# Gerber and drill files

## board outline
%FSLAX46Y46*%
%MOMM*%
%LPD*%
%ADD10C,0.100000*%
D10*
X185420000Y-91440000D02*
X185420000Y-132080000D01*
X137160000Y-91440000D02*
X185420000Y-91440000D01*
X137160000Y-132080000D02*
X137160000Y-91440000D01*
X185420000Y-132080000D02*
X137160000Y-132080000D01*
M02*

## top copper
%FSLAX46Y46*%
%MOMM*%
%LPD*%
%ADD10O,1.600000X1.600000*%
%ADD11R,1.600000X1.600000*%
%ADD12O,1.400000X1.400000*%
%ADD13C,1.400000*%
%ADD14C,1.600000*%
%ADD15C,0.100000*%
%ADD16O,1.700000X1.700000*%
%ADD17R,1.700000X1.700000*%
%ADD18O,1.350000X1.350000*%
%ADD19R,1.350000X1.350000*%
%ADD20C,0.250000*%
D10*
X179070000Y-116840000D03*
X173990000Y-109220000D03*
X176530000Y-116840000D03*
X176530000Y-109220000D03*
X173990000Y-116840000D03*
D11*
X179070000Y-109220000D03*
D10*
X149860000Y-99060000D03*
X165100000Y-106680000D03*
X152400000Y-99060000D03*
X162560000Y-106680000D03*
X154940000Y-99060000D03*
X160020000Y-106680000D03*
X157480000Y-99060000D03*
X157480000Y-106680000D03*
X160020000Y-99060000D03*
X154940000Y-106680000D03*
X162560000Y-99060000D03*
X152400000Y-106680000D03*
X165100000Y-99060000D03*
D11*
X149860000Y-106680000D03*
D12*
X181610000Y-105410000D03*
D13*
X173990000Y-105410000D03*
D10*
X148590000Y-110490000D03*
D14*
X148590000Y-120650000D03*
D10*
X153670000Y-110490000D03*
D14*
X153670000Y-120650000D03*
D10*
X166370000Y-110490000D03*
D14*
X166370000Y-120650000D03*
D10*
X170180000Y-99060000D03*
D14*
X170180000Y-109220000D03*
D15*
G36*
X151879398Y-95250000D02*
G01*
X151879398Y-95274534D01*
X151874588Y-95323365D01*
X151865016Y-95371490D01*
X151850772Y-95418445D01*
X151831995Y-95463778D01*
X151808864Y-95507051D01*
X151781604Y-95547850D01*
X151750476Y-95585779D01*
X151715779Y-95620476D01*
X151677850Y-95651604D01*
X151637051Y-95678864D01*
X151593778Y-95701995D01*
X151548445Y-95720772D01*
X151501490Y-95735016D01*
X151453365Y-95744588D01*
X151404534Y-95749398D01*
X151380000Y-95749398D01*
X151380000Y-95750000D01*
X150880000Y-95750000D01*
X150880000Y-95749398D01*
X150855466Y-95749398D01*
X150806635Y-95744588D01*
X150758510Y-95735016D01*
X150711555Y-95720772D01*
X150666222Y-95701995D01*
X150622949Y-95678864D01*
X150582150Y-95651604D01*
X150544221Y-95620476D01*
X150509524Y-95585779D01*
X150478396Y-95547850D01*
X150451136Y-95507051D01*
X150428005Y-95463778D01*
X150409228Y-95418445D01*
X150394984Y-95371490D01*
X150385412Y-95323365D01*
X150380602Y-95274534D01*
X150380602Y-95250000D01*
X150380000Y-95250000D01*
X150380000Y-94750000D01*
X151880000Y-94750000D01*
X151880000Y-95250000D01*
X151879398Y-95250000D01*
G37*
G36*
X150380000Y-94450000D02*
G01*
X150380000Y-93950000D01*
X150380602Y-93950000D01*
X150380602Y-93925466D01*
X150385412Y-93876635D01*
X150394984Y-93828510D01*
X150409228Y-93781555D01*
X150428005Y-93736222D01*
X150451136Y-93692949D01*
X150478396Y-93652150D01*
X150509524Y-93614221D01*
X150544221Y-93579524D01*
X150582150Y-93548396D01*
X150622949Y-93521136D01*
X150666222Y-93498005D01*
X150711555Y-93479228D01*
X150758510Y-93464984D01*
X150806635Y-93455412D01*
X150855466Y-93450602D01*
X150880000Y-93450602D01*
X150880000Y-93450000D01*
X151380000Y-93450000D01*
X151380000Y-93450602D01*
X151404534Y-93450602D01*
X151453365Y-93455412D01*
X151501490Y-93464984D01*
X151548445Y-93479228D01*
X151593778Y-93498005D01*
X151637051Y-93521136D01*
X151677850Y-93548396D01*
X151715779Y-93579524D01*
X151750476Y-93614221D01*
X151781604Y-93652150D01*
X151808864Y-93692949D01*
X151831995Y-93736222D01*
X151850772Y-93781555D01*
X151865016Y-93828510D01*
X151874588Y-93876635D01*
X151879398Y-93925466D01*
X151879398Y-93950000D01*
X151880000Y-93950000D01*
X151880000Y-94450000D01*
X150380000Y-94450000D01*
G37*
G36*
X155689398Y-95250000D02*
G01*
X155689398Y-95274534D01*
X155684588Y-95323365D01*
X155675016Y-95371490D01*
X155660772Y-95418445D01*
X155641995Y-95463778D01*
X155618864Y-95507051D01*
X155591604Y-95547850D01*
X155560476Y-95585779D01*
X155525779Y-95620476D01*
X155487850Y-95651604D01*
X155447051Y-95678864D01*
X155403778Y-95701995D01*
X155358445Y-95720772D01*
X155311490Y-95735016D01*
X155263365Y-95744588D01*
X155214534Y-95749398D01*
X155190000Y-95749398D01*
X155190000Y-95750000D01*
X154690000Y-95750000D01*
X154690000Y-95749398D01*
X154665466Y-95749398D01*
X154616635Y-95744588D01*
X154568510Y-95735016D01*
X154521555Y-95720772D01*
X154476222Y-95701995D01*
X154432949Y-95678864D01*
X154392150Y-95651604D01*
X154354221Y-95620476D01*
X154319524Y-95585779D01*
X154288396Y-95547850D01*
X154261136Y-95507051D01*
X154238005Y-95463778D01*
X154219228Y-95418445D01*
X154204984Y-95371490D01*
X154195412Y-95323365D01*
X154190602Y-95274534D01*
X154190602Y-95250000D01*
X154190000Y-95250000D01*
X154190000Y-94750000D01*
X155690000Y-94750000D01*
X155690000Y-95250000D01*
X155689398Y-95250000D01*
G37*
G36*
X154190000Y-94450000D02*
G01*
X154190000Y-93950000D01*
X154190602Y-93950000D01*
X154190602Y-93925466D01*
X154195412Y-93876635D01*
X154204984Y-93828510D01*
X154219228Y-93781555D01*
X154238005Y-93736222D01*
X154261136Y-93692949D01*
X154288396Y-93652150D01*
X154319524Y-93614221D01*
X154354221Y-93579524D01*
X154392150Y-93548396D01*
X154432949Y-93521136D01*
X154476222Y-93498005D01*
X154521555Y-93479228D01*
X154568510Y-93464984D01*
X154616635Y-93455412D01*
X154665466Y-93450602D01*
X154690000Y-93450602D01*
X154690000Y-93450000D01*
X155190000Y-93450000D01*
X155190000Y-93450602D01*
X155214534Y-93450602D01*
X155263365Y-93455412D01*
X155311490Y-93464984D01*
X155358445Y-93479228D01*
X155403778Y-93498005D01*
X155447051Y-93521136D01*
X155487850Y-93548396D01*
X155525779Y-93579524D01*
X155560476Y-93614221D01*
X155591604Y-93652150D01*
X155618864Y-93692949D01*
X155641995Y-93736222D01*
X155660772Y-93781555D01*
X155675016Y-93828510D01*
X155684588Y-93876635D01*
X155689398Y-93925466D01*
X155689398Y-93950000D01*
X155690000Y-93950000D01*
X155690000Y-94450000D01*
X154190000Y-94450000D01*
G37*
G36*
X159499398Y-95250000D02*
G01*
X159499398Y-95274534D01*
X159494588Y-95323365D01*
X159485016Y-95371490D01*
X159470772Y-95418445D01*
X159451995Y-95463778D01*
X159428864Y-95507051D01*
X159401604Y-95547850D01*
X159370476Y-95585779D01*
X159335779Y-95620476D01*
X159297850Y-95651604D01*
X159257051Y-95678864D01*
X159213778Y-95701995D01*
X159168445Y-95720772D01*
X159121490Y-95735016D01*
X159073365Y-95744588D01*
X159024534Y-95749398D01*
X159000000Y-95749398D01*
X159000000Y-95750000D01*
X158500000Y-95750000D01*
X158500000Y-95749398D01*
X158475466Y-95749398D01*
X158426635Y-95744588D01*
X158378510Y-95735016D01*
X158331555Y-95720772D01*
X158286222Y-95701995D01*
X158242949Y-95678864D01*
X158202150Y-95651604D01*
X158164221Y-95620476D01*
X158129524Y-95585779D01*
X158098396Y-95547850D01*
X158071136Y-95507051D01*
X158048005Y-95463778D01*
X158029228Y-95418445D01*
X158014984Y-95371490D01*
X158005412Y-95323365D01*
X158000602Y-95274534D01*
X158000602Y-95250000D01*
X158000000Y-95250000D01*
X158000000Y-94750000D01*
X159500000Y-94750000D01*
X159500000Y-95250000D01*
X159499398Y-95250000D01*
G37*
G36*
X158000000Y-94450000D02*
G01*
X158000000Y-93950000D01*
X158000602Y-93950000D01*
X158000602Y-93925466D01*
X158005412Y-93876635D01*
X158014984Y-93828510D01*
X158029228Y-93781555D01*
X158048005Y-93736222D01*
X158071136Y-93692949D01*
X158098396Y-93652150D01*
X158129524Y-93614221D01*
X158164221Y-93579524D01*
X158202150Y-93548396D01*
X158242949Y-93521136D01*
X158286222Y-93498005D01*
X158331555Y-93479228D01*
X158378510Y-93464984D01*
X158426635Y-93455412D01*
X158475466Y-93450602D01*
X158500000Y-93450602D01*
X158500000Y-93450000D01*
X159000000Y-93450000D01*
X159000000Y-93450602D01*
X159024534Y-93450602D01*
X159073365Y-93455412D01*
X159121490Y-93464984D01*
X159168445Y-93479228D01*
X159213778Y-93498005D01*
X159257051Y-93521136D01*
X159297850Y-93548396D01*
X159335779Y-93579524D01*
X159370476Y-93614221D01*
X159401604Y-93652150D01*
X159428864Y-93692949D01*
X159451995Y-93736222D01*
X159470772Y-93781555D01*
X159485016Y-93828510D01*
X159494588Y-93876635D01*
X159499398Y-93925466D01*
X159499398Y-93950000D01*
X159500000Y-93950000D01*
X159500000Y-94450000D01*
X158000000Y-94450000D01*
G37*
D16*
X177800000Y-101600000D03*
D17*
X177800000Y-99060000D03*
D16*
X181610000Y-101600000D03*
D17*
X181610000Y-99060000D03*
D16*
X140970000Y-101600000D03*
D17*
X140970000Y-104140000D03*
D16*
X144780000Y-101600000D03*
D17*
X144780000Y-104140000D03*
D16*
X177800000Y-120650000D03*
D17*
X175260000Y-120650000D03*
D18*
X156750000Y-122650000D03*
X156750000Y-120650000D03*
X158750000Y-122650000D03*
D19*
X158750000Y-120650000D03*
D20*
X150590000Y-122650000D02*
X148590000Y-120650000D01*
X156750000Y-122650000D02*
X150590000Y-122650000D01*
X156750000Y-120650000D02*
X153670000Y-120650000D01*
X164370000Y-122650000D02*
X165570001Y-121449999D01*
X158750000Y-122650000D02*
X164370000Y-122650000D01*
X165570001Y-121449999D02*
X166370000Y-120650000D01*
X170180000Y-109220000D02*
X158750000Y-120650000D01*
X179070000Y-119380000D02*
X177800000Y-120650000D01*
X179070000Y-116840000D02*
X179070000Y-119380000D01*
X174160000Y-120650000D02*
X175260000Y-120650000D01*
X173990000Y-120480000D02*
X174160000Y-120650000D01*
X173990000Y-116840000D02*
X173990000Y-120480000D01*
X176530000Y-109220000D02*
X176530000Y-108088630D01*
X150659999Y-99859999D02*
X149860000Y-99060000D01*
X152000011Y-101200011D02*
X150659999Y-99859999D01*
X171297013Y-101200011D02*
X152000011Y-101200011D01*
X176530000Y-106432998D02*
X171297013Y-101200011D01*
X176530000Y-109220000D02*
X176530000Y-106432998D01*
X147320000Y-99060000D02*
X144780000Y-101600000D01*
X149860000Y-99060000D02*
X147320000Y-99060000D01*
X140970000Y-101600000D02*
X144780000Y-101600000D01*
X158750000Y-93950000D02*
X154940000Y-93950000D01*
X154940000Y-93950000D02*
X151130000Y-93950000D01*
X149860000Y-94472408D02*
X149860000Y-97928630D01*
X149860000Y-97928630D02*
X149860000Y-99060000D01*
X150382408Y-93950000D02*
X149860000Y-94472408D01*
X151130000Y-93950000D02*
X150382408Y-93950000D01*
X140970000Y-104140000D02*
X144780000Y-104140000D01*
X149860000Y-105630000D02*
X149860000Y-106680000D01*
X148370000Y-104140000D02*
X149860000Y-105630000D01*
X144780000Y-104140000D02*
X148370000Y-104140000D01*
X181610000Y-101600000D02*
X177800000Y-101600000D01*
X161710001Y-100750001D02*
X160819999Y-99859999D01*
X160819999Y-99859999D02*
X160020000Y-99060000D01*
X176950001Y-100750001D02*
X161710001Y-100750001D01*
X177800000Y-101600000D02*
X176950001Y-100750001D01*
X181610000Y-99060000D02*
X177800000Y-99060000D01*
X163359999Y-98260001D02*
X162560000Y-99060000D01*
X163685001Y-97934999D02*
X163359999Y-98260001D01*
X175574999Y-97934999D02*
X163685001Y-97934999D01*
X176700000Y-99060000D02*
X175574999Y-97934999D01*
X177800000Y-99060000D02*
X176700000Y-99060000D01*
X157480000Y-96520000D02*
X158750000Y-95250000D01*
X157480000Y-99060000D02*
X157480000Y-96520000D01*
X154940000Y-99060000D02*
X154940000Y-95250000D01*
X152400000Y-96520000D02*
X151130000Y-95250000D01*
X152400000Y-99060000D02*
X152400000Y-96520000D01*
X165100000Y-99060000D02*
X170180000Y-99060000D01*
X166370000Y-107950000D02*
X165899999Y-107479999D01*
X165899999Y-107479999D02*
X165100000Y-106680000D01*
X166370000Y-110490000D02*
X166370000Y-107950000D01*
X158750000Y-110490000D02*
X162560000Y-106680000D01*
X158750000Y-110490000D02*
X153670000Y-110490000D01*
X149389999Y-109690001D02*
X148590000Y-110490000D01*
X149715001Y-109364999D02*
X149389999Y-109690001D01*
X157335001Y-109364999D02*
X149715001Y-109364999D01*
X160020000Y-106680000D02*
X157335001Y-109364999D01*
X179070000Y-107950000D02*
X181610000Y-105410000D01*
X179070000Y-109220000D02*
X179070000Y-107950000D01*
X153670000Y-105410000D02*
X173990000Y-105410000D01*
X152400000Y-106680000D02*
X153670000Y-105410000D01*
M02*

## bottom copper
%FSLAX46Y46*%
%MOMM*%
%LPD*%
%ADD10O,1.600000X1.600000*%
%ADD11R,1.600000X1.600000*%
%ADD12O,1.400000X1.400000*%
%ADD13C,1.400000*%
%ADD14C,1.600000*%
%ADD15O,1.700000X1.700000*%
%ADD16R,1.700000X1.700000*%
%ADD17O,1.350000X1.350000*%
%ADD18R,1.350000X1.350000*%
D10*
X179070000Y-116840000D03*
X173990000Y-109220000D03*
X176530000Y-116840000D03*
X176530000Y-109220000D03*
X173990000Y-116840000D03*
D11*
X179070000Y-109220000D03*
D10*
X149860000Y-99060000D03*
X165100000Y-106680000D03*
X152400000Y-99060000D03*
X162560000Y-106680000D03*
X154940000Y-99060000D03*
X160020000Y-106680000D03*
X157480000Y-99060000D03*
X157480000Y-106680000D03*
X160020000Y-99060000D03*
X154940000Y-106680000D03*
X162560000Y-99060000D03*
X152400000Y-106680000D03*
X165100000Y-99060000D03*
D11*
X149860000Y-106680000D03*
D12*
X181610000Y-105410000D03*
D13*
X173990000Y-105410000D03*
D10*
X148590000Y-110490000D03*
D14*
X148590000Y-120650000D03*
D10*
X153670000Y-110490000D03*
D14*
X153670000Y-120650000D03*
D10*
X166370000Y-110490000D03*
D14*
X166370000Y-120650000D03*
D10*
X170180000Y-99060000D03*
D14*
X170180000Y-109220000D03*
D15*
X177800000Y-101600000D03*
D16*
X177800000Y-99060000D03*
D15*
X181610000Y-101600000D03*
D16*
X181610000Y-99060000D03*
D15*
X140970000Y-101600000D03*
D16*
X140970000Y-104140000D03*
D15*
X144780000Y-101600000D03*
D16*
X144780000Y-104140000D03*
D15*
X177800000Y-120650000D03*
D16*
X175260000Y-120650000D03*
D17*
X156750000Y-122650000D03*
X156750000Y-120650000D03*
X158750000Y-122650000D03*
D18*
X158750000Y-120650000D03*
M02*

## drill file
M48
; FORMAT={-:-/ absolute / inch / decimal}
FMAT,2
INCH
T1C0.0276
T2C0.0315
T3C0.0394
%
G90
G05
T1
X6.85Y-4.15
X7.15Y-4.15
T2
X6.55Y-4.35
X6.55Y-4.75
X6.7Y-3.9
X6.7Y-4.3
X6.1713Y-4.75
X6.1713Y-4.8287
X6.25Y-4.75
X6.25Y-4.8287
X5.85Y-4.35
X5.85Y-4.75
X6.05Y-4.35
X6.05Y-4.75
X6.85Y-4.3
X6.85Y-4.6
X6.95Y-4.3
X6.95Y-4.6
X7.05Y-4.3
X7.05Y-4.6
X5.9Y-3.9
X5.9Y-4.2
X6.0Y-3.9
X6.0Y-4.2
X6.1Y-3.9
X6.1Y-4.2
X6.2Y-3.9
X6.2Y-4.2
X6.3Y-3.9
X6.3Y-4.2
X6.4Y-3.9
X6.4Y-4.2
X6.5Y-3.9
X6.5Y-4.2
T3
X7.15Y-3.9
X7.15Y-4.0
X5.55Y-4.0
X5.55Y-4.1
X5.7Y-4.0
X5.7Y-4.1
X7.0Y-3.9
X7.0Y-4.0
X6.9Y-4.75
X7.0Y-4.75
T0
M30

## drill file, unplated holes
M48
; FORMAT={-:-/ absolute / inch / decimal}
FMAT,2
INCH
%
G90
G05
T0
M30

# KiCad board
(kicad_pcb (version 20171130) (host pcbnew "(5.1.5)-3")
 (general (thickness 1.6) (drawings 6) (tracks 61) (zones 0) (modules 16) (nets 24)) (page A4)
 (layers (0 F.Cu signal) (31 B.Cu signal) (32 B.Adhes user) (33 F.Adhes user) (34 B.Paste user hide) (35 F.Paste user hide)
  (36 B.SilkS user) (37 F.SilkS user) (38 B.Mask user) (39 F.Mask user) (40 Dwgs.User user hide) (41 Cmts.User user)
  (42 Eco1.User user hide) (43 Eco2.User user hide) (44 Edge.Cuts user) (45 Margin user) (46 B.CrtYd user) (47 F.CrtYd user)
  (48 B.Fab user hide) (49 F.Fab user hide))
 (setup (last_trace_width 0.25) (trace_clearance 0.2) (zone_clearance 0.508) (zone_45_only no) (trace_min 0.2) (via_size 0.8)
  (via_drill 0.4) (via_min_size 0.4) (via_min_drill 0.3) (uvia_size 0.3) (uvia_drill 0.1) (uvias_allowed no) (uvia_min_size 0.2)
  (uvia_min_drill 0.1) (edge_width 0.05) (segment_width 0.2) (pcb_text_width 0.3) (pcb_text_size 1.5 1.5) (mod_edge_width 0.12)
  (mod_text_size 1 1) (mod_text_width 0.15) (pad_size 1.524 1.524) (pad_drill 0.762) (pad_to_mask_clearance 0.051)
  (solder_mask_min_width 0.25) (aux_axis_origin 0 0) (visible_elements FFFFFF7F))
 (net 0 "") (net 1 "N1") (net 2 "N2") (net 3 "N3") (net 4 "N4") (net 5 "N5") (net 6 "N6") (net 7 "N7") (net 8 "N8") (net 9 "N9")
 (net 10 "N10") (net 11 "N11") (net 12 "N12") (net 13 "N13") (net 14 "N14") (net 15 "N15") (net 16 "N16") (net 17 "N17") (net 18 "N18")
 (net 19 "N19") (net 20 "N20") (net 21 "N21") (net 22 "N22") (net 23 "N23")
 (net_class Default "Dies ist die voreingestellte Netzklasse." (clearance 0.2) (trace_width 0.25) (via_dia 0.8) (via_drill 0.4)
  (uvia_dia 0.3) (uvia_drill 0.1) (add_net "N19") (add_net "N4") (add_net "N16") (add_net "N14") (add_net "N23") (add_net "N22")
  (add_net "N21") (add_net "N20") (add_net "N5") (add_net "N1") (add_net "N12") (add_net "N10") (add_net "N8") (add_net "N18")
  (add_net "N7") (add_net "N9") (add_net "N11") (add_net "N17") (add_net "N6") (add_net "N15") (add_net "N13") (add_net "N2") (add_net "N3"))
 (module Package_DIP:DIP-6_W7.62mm (layer F.Cu) (at 179.07 109.22 270)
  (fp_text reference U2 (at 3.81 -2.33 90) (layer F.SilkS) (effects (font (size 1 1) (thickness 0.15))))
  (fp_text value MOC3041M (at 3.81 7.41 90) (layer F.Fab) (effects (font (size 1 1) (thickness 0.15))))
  (pad 6 thru_hole oval (at 7.62 0 270) (size 1.6 1.6) (drill 0.8) (layers *.Cu *.Mask) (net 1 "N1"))
  (pad 3 thru_hole oval (at 0 5.08 270) (size 1.6 1.6) (drill 0.8) (layers *.Cu *.Mask) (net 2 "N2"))
  (pad 5 thru_hole oval (at 7.62 2.54 270) (size 1.6 1.6) (drill 0.8) (layers *.Cu *.Mask) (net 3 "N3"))
  (pad 2 thru_hole oval (at 0 2.54 270) (size 1.6 1.6) (drill 0.8) (layers *.Cu *.Mask) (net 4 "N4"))
  (pad 4 thru_hole oval (at 7.62 5.08 270) (size 1.6 1.6) (drill 0.8) (layers *.Cu *.Mask) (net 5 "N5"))
  (pad 1 thru_hole rect (at 0 0 270) (size 1.6 1.6) (drill 0.8) (layers *.Cu *.Mask) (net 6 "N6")))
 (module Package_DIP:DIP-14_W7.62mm (layer F.Cu) (at 149.86 106.68 90)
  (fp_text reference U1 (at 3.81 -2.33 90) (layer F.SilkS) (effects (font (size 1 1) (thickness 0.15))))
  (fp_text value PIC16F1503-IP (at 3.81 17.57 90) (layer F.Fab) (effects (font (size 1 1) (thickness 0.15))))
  (pad 14 thru_hole oval (at 7.62 0 90) (size 1.6 1.6) (drill 0.8) (layers *.Cu *.Mask) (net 4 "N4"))
  (pad 7 thru_hole oval (at 0 15.24 90) (size 1.6 1.6) (drill 0.8) (layers *.Cu *.Mask) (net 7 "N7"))
  (pad 13 thru_hole oval (at 7.62 2.54 90) (size 1.6 1.6) (drill 0.8) (layers *.Cu *.Mask) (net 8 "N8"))
  (pad 6 thru_hole oval (at 0 12.7 90) (size 1.6 1.6) (drill 0.8) (layers *.Cu *.Mask) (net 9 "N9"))
  (pad 12 thru_hole oval (at 7.62 5.08 90) (size 1.6 1.6) (drill 0.8) (layers *.Cu *.Mask) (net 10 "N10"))
  (pad 5 thru_hole oval (at 0 10.16 90) (size 1.6 1.6) (drill 0.8) (layers *.Cu *.Mask) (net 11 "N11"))
  (pad 11 thru_hole oval (at 7.62 7.62 90) (size 1.6 1.6) (drill 0.8) (layers *.Cu *.Mask) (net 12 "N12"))
  (pad 4 thru_hole oval (at 0 7.62 90) (size 1.6 1.6) (drill 0.8) (layers *.Cu *.Mask) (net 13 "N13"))
  (pad 10 thru_hole oval (at 7.62 10.16 90) (size 1.6 1.6) (drill 0.8) (layers *.Cu *.Mask) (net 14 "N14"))
  (pad 3 thru_hole oval (at 0 5.08 90) (size 1.6 1.6) (drill 0.8) (layers *.Cu *.Mask) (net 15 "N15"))
  (pad 9 thru_hole oval (at 7.62 12.7 90) (size 1.6 1.6) (drill 0.8) (layers *.Cu *.Mask) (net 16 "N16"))
  (pad 2 thru_hole oval (at 0 2.54 90) (size 1.6 1.6) (drill 0.8) (layers *.Cu *.Mask) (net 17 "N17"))
  (pad 8 thru_hole oval (at 7.62 15.24 90) (size 1.6 1.6) (drill 0.8) (layers *.Cu *.Mask) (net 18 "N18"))
  (pad 1 thru_hole rect (at 0 0 90) (size 1.6 1.6) (drill 0.8) (layers *.Cu *.Mask) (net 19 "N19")))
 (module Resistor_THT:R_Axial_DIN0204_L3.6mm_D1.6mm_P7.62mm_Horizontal (layer F.Cu) (at 173.99 105.41)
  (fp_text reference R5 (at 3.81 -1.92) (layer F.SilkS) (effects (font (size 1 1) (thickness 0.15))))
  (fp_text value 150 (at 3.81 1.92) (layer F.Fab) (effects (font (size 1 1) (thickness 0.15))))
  (pad 2 thru_hole oval (at 7.62 0) (size 1.4 1.4) (drill 0.7) (layers *.Cu *.Mask) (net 6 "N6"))
  (pad 1 thru_hole circle (at 0 0) (size 1.4 1.4) (drill 0.7) (layers *.Cu *.Mask) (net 17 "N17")))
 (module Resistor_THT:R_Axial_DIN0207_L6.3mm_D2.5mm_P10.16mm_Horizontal (layer F.Cu) (at 148.59 120.65 90)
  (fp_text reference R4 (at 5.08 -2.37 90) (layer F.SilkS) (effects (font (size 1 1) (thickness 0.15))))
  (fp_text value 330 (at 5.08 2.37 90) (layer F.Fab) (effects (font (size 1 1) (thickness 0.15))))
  (pad 2 thru_hole oval (at 10.16 0 90) (size 1.6 1.6) (drill 0.8) (layers *.Cu *.Mask) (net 11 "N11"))
  (pad 1 thru_hole circle (at 0 0 90) (size 1.6 1.6) (drill 0.8) (layers *.Cu *.Mask) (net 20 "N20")))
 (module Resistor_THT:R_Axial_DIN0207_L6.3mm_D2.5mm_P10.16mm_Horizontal (layer F.Cu) (at 153.67 120.65 90)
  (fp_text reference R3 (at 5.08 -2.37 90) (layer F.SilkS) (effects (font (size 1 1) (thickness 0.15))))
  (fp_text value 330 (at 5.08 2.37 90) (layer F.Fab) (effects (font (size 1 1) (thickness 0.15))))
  (pad 2 thru_hole oval (at 10.16 0 90) (size 1.6 1.6) (drill 0.8) (layers *.Cu *.Mask) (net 9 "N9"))
  (pad 1 thru_hole circle (at 0 0 90) (size 1.6 1.6) (drill 0.8) (layers *.Cu *.Mask) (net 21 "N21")))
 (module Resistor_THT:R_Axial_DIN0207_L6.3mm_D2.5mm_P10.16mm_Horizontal (layer F.Cu) (at 166.37 120.65 90)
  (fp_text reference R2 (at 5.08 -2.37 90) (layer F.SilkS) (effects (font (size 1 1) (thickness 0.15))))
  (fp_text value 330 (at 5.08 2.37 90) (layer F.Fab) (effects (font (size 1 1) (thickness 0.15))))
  (pad 2 thru_hole oval (at 10.16 0 90) (size 1.6 1.6) (drill 0.8) (layers *.Cu *.Mask) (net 7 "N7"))
  (pad 1 thru_hole circle (at 0 0 90) (size 1.6 1.6) (drill 0.8) (layers *.Cu *.Mask) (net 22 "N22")))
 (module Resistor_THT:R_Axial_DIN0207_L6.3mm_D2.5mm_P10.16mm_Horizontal (layer F.Cu) (at 170.18 109.22 90)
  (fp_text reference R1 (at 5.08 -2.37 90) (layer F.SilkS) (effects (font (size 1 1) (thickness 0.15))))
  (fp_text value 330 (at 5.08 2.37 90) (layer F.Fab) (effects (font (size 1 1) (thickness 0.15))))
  (pad 2 thru_hole oval (at 10.16 0 90) (size 1.6 1.6) (drill 0.8) (layers *.Cu *.Mask) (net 18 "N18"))
  (pad 1 thru_hole circle (at 0 0 90) (size 1.6 1.6) (drill 0.8) (layers *.Cu *.Mask) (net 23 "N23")))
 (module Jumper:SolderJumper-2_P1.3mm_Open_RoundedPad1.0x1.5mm (layer F.Cu) (at 151.13 94.6 270)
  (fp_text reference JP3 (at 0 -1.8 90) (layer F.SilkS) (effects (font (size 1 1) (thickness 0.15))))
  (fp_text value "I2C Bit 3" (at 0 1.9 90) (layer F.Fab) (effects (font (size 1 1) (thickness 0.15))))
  (pad 2 smd custom (at 0.65 0 270) (size 1 0.5) (layers F.Cu F.Mask) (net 8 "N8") (zone_connect 2)
   (options (clearance outline) (anchor rect)) (primitives))
  (pad 1 smd custom (at -0.65 0 270) (size 1 0.5) (layers F.Cu F.Mask) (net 4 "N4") (zone_connect 2)
   (options (clearance outline) (anchor rect)) (primitives)))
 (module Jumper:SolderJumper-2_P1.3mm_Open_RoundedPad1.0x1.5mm (layer F.Cu) (at 154.94 94.6 270)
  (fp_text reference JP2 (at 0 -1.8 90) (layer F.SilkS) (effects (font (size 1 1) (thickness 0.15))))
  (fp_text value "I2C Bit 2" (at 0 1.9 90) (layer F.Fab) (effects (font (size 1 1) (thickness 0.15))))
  (pad 2 smd custom (at 0.65 0 270) (size 1 0.5) (layers F.Cu F.Mask) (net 10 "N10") (zone_connect 2)
   (options (clearance outline) (anchor rect)) (primitives))
  (pad 1 smd custom (at -0.65 0 270) (size 1 0.5) (layers F.Cu F.Mask) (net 4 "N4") (zone_connect 2)
   (options (clearance outline) (anchor rect)) (primitives)))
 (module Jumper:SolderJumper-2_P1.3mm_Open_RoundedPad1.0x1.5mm (layer F.Cu) (at 158.75 94.6 270)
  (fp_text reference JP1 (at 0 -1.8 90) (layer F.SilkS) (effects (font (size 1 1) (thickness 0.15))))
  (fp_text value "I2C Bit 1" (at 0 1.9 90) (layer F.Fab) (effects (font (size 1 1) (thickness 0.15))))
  (pad 2 smd custom (at 0.65 0 270) (size 1 0.5) (layers F.Cu F.Mask) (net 12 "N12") (zone_connect 2)
   (options (clearance outline) (anchor rect)) (primitives))
  (pad 1 smd custom (at -0.65 0 270) (size 1 0.5) (layers F.Cu F.Mask) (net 4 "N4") (zone_connect 2)
   (options (clearance outline) (anchor rect)) (primitives)))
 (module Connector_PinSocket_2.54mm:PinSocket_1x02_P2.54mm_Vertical (layer F.Cu) (at 177.8 99.06)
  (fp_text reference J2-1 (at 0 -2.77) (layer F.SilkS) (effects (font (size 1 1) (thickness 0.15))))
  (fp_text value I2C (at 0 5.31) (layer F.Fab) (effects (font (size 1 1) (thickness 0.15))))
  (pad 2 thru_hole oval (at 0 2.54) (size 1.7 1.7) (drill 1) (layers *.Cu *.Mask) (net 14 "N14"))
  (pad 1 thru_hole rect (at 0 0) (size 1.7 1.7) (drill 1) (layers *.Cu *.Mask) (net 16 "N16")))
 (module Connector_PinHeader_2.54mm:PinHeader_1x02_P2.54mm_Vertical (layer B.Cu) (at 181.61 99.06 180)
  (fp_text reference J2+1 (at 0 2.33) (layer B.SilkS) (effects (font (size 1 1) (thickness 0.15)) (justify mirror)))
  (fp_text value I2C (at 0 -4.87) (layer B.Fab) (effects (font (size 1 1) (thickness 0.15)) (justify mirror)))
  (pad 2 thru_hole oval (at 0 -2.54 180) (size 1.7 1.7) (drill 1) (layers *.Cu *.Mask) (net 14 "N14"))
  (pad 1 thru_hole rect (at 0 0 180) (size 1.7 1.7) (drill 1) (layers *.Cu *.Mask) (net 16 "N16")))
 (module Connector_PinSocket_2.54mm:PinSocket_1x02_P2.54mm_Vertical (layer F.Cu) (at 140.97 104.14 180)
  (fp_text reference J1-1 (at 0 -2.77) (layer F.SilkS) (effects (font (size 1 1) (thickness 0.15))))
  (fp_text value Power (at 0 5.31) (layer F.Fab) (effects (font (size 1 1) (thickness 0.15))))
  (pad 2 thru_hole oval (at 0 2.54 180) (size 1.7 1.7) (drill 1) (layers *.Cu *.Mask) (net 4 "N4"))
  (pad 1 thru_hole rect (at 0 0 180) (size 1.7 1.7) (drill 1) (layers *.Cu *.Mask) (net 19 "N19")))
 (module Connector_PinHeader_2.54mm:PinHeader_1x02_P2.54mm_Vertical (layer B.Cu) (at 144.78 104.14)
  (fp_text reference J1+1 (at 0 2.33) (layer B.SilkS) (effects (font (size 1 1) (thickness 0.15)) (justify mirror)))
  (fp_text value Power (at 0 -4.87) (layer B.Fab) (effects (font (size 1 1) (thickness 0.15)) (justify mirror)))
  (pad 2 thru_hole oval (at 0 -2.54) (size 1.7 1.7) (drill 1) (layers *.Cu *.Mask) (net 4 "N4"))
  (pad 1 thru_hole rect (at 0 0) (size 1.7 1.7) (drill 1) (layers *.Cu *.Mask) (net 19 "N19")))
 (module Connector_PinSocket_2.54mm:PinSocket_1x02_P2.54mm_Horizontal (layer F.Cu) (at 175.26 120.65 90)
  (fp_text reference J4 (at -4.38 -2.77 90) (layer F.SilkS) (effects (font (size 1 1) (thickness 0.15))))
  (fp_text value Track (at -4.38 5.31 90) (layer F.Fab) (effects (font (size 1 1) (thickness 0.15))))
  (pad 2 thru_hole oval (at 0 2.54 90) (size 1.7 1.7) (drill 1) (layers *.Cu *.Mask) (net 1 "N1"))
  (pad 1 thru_hole rect (at 0 0 90) (size 1.7 1.7) (drill 1) (layers *.Cu *.Mask) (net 5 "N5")))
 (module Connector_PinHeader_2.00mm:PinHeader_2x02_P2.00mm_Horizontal (layer F.Cu) (at 158.75 120.65 270)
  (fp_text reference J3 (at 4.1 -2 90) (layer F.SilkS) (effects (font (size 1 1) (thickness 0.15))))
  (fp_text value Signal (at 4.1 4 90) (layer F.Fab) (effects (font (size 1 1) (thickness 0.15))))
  (pad 4 thru_hole oval (at 2 2 270) (size 1.35 1.35) (drill 0.8) (layers *.Cu *.Mask) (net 20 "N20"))
  (pad 3 thru_hole oval (at 0 2 270) (size 1.35 1.35) (drill 0.8) (layers *.Cu *.Mask) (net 21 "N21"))
  (pad 2 thru_hole oval (at 2 0 270) (size 1.35 1.35) (drill 0.8) (layers *.Cu *.Mask) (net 22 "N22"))
  (pad 1 thru_hole rect (at 0 0 270) (size 1.35 1.35) (drill 0.8) (layers *.Cu *.Mask) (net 23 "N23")))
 (gr_line (start 185.42 91.44) (end 185.42 132.08) (layer Edge.Cuts) (width 0.1))
 (gr_line (start 137.16 91.44) (end 185.42 91.44) (layer Edge.Cuts) (width 0.1))
 (gr_line (start 137.16 132.08) (end 137.16 91.44) (layer Edge.Cuts) (width 0.1))
 (gr_line (start 185.42 132.08) (end 137.16 132.08) (layer Edge.Cuts) (width 0.1))
 (segment (start 150.59 122.65) (end 148.59 120.65) (width 0.25) (layer F.Cu) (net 20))
 (segment (start 156.75 122.65) (end 150.59 122.65) (width 0.25) (layer F.Cu) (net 20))
 (segment (start 156.75 120.65) (end 153.67 120.65) (width 0.25) (layer F.Cu) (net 21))
 (segment (start 164.37 122.65) (end 165.570001 121.449999) (width 0.25) (layer F.Cu) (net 22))
 (segment (start 158.75 122.65) (end 164.37 122.65) (width 0.25) (layer F.Cu) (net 22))
 (segment (start 165.570001 121.449999) (end 166.37 120.65) (width 0.25) (layer F.Cu) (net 22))
 (segment (start 170.18 109.22) (end 158.75 120.65) (width 0.25) (layer F.Cu) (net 23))
 (segment (start 179.07 119.38) (end 177.8 120.65) (width 0.25) (layer F.Cu) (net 1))
 (segment (start 179.07 116.84) (end 179.07 119.38) (width 0.25) (layer F.Cu) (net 1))
 (segment (start 174.16 120.65) (end 175.26 120.65) (width 0.25) (layer F.Cu) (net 5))
 (segment (start 173.99 120.48) (end 174.16 120.65) (width 0.25) (layer F.Cu) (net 5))
 (segment (start 173.99 116.84) (end 173.99 120.48) (width 0.25) (layer F.Cu) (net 5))
 (segment (start 176.53 109.22) (end 176.53 108.08863) (width 0.25) (layer F.Cu) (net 4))
 (segment (start 150.659999 99.859999) (end 149.86 99.06) (width 0.25) (layer F.Cu) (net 4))
 (segment (start 152.000011 101.200011) (end 150.659999 99.859999) (width 0.25) (layer F.Cu) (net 4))
 (segment (start 171.297013 101.200011) (end 152.000011 101.200011) (width 0.25) (layer F.Cu) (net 4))
 (segment (start 176.53 106.432998) (end 171.297013 101.200011) (width 0.25) (layer F.Cu) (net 4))
 (segment (start 176.53 109.22) (end 176.53 106.432998) (width 0.25) (layer F.Cu) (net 4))
 (segment (start 147.32 99.06) (end 144.78 101.6) (width 0.25) (layer F.Cu) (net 4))
 (segment (start 149.86 99.06) (end 147.32 99.06) (width 0.25) (layer F.Cu) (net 4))
 (segment (start 140.97 101.6) (end 144.78 101.6) (width 0.25) (layer F.Cu) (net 4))
 (segment (start 158.75 93.95) (end 154.94 93.95) (width 0.25) (layer F.Cu) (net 4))
 (segment (start 154.94 93.95) (end 151.13 93.95) (width 0.25) (layer F.Cu) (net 4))
 (segment (start 149.86 94.472408) (end 149.86 97.92863) (width 0.25) (layer F.Cu) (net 4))
 (segment (start 149.86 97.92863) (end 149.86 99.06) (width 0.25) (layer F.Cu) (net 4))
 (segment (start 150.382408 93.95) (end 149.86 94.472408) (width 0.25) (layer F.Cu) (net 4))
 (segment (start 151.13 93.95) (end 150.382408 93.95) (width 0.25) (layer F.Cu) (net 4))
 (segment (start 140.97 104.14) (end 144.78 104.14) (width 0.25) (layer F.Cu) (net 19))
 (segment (start 149.86 105.63) (end 149.86 106.68) (width 0.25) (layer F.Cu) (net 19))
 (segment (start 148.37 104.14) (end 149.86 105.63) (width 0.25) (layer F.Cu) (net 19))
 (segment (start 144.78 104.14) (end 148.37 104.14) (width 0.25) (layer F.Cu) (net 19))
 (segment (start 181.61 101.6) (end 177.8 101.6) (width 0.25) (layer F.Cu) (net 14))
 (segment (start 161.710001 100.750001) (end 160.819999 99.859999) (width 0.25) (layer F.Cu) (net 14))
 (segment (start 160.819999 99.859999) (end 160.02 99.06) (width 0.25) (layer F.Cu) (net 14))
 (segment (start 176.950001 100.750001) (end 161.710001 100.750001) (width 0.25) (layer F.Cu) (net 14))
 (segment (start 177.8 101.6) (end 176.950001 100.750001) (width 0.25) (layer F.Cu) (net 14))
 (segment (start 181.61 99.06) (end 177.8 99.06) (width 0.25) (layer F.Cu) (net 16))
 (segment (start 163.359999 98.260001) (end 162.56 99.06) (width 0.25) (layer F.Cu) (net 16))
 (segment (start 163.685001 97.934999) (end 163.359999 98.260001) (width 0.25) (layer F.Cu) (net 16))
 (segment (start 175.574999 97.934999) (end 163.685001 97.934999) (width 0.25) (layer F.Cu) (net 16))
 (segment (start 176.7 99.06) (end 175.574999 97.934999) (width 0.25) (layer F.Cu) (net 16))
 (segment (start 177.8 99.06) (end 176.7 99.06) (width 0.25) (layer F.Cu) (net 16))
 (segment (start 157.48 96.52) (end 158.75 95.25) (width 0.25) (layer F.Cu) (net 12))
 (segment (start 157.48 99.06) (end 157.48 96.52) (width 0.25) (layer F.Cu) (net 12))
 (segment (start 154.94 99.06) (end 154.94 95.25) (width 0.25) (layer F.Cu) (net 10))
 (segment (start 152.4 96.52) (end 151.13 95.25) (width 0.25) (layer F.Cu) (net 8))
 (segment (start 152.4 99.06) (end 152.4 96.52) (width 0.25) (layer F.Cu) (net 8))
 (segment (start 165.1 99.06) (end 170.18 99.06) (width 0.25) (layer F.Cu) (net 18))
 (segment (start 166.37 107.95) (end 165.899999 107.479999) (width 0.25) (layer F.Cu) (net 7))
 (segment (start 165.899999 107.479999) (end 165.1 106.68) (width 0.25) (layer F.Cu) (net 7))
 (segment (start 166.37 110.49) (end 166.37 107.95) (width 0.25) (layer F.Cu) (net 7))
 (segment (start 158.75 110.49) (end 162.56 106.68) (width 0.25) (layer F.Cu) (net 9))
 (segment (start 158.75 110.49) (end 153.67 110.49) (width 0.25) (layer F.Cu) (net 9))
 (segment (start 149.389999 109.690001) (end 148.59 110.49) (width 0.25) (layer F.Cu) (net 11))
 (segment (start 149.715001 109.364999) (end 149.389999 109.690001) (width 0.25) (layer F.Cu) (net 11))
 (segment (start 157.335001 109.364999) (end 149.715001 109.364999) (width 0.25) (layer F.Cu) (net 11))
 (segment (start 160.02 106.68) (end 157.335001 109.364999) (width 0.25) (layer F.Cu) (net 11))
 (segment (start 179.07 107.95) (end 181.61 105.41) (width 0.25) (layer F.Cu) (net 6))
 (segment (start 179.07 109.22) (end 179.07 107.95) (width 0.25) (layer F.Cu) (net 6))
 (segment (start 153.67 105.41) (end 173.99 105.41) (width 0.25) (layer F.Cu) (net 17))
 (segment (start 152.4 106.68) (end 153.67 105.41) (width 0.25) (layer F.Cu) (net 17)))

